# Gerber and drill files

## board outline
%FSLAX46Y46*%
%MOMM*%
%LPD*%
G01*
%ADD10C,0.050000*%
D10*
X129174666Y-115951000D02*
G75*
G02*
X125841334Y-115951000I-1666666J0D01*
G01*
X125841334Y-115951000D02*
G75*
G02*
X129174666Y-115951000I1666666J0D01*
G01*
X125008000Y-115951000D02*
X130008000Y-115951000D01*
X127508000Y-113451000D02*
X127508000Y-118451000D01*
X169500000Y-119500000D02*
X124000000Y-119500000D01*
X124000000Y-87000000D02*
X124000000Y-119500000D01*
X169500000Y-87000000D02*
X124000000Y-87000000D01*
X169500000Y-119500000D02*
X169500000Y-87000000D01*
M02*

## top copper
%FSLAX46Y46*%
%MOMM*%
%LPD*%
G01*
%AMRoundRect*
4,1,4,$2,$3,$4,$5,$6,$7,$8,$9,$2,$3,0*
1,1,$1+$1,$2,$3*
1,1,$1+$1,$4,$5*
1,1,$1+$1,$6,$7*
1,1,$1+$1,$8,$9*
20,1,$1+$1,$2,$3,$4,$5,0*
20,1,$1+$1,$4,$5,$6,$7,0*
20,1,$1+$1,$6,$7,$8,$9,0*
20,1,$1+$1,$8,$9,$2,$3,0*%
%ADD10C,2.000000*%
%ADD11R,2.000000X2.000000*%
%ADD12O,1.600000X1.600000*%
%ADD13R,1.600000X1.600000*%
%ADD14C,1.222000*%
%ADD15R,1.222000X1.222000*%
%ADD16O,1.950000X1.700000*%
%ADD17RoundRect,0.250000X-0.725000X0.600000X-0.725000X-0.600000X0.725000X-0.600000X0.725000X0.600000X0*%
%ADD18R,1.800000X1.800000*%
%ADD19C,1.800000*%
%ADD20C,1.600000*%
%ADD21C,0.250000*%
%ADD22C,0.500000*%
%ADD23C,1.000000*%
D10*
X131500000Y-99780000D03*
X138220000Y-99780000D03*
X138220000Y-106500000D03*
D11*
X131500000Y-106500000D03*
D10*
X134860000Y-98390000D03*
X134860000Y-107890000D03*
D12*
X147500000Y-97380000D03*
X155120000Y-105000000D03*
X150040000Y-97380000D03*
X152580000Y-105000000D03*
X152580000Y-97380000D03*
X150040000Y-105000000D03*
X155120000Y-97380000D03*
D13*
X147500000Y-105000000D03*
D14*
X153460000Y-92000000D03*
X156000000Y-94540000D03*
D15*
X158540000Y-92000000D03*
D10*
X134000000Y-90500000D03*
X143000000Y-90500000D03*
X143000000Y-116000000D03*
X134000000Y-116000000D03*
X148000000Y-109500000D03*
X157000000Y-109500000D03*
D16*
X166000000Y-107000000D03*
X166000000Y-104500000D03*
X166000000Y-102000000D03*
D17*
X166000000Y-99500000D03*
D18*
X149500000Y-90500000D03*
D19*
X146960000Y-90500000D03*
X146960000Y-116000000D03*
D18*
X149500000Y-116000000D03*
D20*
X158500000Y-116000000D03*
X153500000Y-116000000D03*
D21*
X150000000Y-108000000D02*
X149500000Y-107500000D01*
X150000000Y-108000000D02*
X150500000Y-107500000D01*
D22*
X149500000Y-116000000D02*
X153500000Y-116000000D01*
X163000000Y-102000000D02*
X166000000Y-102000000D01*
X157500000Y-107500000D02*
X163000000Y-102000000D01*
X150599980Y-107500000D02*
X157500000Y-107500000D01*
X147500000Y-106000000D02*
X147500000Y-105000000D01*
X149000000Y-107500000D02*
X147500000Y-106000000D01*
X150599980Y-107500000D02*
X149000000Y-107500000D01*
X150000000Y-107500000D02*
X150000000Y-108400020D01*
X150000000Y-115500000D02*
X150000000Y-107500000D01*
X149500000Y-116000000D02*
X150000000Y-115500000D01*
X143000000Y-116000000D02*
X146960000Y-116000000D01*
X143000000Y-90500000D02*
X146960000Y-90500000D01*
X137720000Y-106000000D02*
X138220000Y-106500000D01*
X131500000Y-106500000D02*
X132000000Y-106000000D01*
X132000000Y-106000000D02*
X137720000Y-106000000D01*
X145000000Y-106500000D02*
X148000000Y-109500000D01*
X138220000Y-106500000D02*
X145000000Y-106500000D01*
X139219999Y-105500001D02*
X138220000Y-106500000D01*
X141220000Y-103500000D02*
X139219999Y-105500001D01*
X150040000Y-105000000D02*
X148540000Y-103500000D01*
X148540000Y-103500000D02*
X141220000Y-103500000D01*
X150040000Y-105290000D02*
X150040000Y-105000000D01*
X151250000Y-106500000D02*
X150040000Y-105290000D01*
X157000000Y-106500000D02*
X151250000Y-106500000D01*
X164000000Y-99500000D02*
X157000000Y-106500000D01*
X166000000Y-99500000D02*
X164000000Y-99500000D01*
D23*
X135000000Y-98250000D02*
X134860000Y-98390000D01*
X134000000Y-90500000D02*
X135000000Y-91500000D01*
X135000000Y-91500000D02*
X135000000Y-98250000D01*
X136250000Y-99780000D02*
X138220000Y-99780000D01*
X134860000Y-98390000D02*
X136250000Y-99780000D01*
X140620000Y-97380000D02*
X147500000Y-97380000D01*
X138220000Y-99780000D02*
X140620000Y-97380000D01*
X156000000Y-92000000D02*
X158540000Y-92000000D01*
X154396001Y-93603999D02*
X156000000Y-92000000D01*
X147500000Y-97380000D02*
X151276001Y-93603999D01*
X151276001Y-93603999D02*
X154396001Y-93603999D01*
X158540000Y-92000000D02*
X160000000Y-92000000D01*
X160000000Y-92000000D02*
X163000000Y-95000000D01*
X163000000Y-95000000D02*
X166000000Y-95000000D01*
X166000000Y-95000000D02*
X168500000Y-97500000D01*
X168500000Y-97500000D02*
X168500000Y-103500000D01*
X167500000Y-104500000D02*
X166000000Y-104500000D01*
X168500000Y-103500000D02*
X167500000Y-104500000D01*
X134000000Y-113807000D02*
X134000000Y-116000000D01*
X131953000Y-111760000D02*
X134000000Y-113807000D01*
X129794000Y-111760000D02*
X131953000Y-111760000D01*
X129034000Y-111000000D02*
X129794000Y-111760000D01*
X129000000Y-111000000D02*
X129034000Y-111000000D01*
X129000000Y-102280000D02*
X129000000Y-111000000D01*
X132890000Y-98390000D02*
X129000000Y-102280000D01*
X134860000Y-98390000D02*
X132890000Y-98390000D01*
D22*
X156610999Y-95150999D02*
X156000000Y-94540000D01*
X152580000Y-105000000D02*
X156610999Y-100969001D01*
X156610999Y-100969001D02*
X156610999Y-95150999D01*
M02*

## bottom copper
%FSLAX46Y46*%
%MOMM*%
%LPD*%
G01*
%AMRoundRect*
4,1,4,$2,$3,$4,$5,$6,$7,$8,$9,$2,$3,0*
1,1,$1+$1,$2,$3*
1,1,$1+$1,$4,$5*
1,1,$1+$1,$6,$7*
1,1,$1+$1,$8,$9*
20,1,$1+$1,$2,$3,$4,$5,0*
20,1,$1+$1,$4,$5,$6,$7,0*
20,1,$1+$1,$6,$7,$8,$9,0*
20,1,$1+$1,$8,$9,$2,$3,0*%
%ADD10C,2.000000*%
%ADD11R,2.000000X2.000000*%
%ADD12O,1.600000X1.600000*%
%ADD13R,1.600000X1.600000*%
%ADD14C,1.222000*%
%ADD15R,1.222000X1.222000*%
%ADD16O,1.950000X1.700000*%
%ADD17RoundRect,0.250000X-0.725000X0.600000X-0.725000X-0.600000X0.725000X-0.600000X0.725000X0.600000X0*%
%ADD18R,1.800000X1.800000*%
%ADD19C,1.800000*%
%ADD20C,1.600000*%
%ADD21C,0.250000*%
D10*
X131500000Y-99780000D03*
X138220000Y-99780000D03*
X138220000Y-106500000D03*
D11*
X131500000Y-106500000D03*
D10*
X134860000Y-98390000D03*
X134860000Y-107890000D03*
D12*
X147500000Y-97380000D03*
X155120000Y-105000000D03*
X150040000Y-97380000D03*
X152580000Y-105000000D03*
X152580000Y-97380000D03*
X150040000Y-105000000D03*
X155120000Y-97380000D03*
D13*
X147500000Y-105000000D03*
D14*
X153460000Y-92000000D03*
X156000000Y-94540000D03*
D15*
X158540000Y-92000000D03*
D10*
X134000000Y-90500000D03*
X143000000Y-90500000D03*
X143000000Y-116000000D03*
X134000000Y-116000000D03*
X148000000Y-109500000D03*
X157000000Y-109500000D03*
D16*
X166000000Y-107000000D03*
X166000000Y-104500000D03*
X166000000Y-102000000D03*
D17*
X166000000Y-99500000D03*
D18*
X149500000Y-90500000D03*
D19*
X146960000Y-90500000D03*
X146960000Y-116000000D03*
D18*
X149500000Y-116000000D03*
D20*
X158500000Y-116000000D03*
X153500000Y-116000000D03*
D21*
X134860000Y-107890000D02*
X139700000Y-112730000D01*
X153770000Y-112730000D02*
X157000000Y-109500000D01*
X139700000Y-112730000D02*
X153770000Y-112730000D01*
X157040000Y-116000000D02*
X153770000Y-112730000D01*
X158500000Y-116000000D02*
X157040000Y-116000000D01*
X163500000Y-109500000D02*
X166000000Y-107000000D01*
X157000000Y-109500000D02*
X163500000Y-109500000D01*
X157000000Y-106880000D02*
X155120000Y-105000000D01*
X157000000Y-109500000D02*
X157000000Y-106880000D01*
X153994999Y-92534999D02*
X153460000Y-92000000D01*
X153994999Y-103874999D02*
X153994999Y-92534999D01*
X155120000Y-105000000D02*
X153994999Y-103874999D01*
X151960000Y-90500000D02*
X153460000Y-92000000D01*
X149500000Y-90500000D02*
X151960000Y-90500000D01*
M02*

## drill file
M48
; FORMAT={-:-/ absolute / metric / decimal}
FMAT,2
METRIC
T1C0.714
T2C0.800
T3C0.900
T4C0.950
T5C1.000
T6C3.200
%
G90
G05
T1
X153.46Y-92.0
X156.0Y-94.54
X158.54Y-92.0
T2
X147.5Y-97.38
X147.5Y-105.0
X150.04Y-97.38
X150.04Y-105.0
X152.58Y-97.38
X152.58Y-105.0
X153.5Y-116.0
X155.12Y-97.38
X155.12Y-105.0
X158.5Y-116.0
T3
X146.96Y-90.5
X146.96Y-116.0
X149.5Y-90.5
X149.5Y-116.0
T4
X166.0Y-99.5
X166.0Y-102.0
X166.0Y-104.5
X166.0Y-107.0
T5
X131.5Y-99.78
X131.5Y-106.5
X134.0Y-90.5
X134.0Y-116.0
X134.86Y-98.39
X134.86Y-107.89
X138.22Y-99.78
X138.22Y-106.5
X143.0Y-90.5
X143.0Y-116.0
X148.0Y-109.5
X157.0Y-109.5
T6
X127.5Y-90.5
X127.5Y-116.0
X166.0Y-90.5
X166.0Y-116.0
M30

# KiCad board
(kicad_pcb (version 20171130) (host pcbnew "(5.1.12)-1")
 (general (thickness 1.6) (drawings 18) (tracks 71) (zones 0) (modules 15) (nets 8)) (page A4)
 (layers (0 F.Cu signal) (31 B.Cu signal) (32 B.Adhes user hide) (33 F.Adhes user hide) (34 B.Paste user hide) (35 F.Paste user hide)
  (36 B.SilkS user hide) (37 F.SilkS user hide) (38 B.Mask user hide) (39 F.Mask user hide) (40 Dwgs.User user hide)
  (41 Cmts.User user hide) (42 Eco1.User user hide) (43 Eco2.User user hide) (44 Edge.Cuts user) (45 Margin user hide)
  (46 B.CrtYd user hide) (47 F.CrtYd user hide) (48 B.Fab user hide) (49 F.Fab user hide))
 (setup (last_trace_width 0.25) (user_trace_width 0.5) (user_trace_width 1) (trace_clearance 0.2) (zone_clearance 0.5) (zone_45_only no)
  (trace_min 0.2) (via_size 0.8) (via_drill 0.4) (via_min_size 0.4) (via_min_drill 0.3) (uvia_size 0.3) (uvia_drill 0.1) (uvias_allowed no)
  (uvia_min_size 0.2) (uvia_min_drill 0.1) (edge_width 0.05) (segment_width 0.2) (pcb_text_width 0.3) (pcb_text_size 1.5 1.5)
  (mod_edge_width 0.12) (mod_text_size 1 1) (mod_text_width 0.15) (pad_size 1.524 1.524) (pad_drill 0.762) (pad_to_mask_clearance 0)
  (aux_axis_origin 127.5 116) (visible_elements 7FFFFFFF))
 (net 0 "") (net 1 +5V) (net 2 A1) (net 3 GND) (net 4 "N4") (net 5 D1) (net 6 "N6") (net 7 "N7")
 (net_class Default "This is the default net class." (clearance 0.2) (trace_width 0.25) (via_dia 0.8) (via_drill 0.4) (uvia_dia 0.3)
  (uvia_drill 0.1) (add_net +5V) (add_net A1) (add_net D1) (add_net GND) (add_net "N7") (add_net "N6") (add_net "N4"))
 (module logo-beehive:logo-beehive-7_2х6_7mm (layer F.Cu) (at 161 113.5 90)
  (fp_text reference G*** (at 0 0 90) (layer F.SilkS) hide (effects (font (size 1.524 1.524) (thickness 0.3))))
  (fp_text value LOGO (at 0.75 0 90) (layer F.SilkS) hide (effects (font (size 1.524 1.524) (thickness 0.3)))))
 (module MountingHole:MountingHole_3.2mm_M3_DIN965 (layer F.Cu) (at 166 90.5)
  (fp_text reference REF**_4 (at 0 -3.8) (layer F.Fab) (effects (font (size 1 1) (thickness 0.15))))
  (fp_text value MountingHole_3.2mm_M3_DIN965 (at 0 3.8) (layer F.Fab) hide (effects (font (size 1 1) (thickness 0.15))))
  (pad 1 np_thru_hole circle (at 0 0) (size 3.2 3.2) (drill 3.2) (layers *.Cu *.Mask)))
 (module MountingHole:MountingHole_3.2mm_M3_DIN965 (layer F.Cu) (at 166 116)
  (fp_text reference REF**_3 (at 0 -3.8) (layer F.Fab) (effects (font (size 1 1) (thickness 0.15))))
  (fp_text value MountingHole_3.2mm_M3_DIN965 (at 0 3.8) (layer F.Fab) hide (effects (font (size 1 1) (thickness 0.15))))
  (pad 1 np_thru_hole circle (at 0 0) (size 3.2 3.2) (drill 3.2) (layers *.Cu *.Mask)))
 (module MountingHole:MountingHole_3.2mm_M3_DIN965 (layer F.Cu) (at 127.5 90.5)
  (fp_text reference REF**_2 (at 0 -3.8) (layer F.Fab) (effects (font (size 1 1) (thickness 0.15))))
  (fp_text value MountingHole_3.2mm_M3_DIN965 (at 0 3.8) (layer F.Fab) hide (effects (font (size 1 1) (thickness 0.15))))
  (pad 1 np_thru_hole circle (at 0 0) (size 3.2 3.2) (drill 3.2) (layers *.Cu *.Mask)))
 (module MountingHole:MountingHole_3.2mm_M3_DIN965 (layer F.Cu) (at 127.5 116)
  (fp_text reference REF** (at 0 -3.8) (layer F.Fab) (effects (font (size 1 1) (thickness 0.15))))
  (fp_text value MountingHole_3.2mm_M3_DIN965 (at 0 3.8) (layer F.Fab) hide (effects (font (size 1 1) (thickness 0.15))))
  (pad 1 np_thru_hole circle (at 0 0) (size 3.2 3.2) (drill 3.2) (layers *.Cu *.Mask)))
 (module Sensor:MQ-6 (layer F.Cu) (at 131.5 106.5 90)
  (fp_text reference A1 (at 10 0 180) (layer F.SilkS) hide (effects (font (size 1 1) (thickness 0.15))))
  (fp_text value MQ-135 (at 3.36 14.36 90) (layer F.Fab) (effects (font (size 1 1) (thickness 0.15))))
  (pad 6 thru_hole circle (at 6.72 0) (size 2 2) (drill 1) (layers *.Cu *.Mask) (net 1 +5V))
  (pad 4 thru_hole circle (at 6.72 6.72 270) (size 2 2) (drill 1) (layers *.Cu *.Mask) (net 1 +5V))
  (pad 3 thru_hole circle (at 0 6.72 180) (size 2 2) (drill 1) (layers *.Cu *.Mask) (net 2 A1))
  (pad 1 thru_hole rect (at 0 0 90) (size 2 2) (drill 1) (layers *.Cu *.Mask) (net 2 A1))
  (pad 5 thru_hole circle (at 8.11 3.36 90) (size 2 2) (drill 1) (layers *.Cu *.Mask) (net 1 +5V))
  (pad 2 thru_hole circle (at -1.39 3.36 90) (size 2 2) (drill 1) (layers *.Cu *.Mask) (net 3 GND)))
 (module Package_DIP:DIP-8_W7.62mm (layer F.Cu) (at 147.5 105 90)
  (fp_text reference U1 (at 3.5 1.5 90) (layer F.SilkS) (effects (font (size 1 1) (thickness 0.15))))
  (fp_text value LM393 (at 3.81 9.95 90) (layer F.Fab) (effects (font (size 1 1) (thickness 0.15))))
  (pad 8 thru_hole oval (at 7.62 0 90) (size 1.6 1.6) (drill 0.8) (layers *.Cu *.Mask) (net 1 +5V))
  (pad 4 thru_hole oval (at 0 7.62 90) (size 1.6 1.6) (drill 0.8) (layers *.Cu *.Mask) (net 3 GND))
  (pad 7 thru_hole oval (at 7.62 2.54 90) (size 1.6 1.6) (drill 0.8) (layers *.Cu *.Mask))
  (pad 3 thru_hole oval (at 0 5.08 90) (size 1.6 1.6) (drill 0.8) (layers *.Cu *.Mask) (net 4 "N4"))
  (pad 6 thru_hole oval (at 7.62 5.08 90) (size 1.6 1.6) (drill 0.8) (layers *.Cu *.Mask))
  (pad 2 thru_hole oval (at 0 2.54 90) (size 1.6 1.6) (drill 0.8) (layers *.Cu *.Mask) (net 2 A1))
  (pad 5 thru_hole oval (at 7.62 7.62 90) (size 1.6 1.6) (drill 0.8) (layers *.Cu *.Mask))
  (pad 1 thru_hole rect (at 0 0 90) (size 1.6 1.6) (drill 0.8) (layers *.Cu *.Mask) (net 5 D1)))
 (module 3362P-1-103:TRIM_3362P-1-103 (layer F.Cu) (at 156 92 180)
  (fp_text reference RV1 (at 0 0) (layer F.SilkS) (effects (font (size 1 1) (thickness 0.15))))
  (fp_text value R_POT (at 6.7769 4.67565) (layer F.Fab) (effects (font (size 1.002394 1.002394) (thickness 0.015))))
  (pad 3 thru_hole circle (at 2.54 0 180) (size 1.222 1.222) (drill 0.714) (layers *.Cu *.Mask) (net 3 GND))
  (pad 2 thru_hole circle (at 0 -2.54 180) (size 1.222 1.222) (drill 0.714) (layers *.Cu *.Mask) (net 4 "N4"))
  (pad 1 thru_hole rect (at -2.54 0 180) (size 1.222 1.222) (drill 0.714) (layers *.Cu *.Mask) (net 1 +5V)))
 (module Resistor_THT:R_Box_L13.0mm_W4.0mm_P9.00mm (layer F.Cu) (at 134 90.5)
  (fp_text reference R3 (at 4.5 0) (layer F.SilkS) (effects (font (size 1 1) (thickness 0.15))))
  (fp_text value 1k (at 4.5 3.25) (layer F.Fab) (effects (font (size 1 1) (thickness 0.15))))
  (pad 1 thru_hole circle (at 0 0) (size 2 2) (drill 1) (layers *.Cu *.Mask) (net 1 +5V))
  (pad 2 thru_hole circle (at 9 0) (size 2 2) (drill 1) (layers *.Cu *.Mask) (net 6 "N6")))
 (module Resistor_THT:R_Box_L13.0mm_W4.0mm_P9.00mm (layer F.Cu) (at 134 116)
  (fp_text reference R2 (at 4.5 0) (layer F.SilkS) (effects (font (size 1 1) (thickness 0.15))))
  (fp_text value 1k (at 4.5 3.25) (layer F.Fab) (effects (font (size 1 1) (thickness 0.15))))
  (pad 2 thru_hole circle (at 9 0) (size 2 2) (drill 1) (layers *.Cu *.Mask) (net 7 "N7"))
  (pad 1 thru_hole circle (at 0 0) (size 2 2) (drill 1) (layers *.Cu *.Mask) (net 1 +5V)))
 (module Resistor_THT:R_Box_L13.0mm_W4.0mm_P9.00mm (layer F.Cu) (at 148 109.5)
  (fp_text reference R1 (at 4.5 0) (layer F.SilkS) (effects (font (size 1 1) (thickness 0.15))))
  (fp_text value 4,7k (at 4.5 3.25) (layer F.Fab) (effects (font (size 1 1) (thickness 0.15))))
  (pad 1 thru_hole circle (at 0 0) (size 2 2) (drill 1) (layers *.Cu *.Mask) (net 2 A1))
  (pad 2 thru_hole circle (at 9 0) (size 2 2) (drill 1) (layers *.Cu *.Mask) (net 3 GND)))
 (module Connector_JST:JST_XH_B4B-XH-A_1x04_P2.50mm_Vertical (layer F.Cu) (at 166 99.5 270)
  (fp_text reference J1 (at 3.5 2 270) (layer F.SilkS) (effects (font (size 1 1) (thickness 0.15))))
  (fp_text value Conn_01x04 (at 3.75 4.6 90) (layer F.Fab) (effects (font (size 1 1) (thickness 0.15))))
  (pad 4 thru_hole oval (at 7.5 0 270) (size 1.7 1.95) (drill 0.95) (layers *.Cu *.Mask) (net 3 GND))
  (pad 3 thru_hole oval (at 5 0 270) (size 1.7 1.95) (drill 0.95) (layers *.Cu *.Mask) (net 1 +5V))
  (pad 2 thru_hole oval (at 2.5 0 270) (size 1.7 1.95) (drill 0.95) (layers *.Cu *.Mask) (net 5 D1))
  (pad 1 thru_hole roundrect (at 0 0 270) (size 1.7 1.95) (drill 0.95) (layers *.Cu *.Mask) (roundrect_rratio 0.1470588235294118) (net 2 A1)))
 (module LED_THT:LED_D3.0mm (layer F.Cu) (at 149.5 90.5 180)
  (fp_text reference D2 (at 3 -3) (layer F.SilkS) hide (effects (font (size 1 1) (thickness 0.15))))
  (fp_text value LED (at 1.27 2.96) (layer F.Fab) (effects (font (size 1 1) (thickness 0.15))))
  (pad 1 thru_hole rect (at 0 0 180) (size 1.8 1.8) (drill 0.9) (layers *.Cu *.Mask) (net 3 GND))
  (pad 2 thru_hole circle (at 2.54 0 180) (size 1.8 1.8) (drill 0.9) (layers *.Cu *.Mask) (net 6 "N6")))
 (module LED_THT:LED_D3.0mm (layer F.Cu) (at 149.5 116 180)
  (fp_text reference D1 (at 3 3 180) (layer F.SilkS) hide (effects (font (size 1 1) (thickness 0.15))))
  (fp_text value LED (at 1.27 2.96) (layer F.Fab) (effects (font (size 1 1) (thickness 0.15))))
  (pad 2 thru_hole circle (at 2.54 0 180) (size 1.8 1.8) (drill 0.9) (layers *.Cu *.Mask) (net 7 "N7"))
  (pad 1 thru_hole rect (at 0 0 180) (size 1.8 1.8) (drill 0.9) (layers *.Cu *.Mask) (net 5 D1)))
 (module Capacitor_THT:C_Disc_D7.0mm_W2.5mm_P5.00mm (layer F.Cu) (at 153.5 116)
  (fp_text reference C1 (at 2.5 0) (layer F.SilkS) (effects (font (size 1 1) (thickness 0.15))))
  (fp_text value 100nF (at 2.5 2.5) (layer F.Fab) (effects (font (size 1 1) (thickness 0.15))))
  (pad 2 thru_hole circle (at 5 0) (size 1.6 1.6) (drill 0.8) (layers *.Cu *.Mask) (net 3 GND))
  (pad 1 thru_hole circle (at 0 0) (size 1.6 1.6) (drill 0.8) (layers *.Cu *.Mask) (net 5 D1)))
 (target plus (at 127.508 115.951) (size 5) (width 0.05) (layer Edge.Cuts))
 (gr_line (start 169.5 119.5) (end 124 119.5) (layer Edge.Cuts) (width 0.05))
 (gr_line (start 124 87) (end 124 119.5) (layer Edge.Cuts) (width 0.05))
 (gr_line (start 169.5 87) (end 124 87) (layer Edge.Cuts) (width 0.05))
 (gr_line (start 169.5 119.5) (end 169.5 87) (layer Edge.Cuts) (width 0.05))
 (segment (start 134.86 107.89) (end 139.7 112.73) (width 0.25) (layer B.Cu) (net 3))
 (segment (start 153.77 112.73) (end 157 109.5) (width 0.25) (layer B.Cu) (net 3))
 (segment (start 139.7 112.73) (end 153.77 112.73) (width 0.25) (layer B.Cu) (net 3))
 (segment (start 157.04 116) (end 153.77 112.73) (width 0.25) (layer B.Cu) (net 3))
 (segment (start 158.5 116) (end 157.04 116) (width 0.25) (layer B.Cu) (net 3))
 (segment (start 163.5 109.5) (end 166 107) (width 0.25) (layer B.Cu) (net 3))
 (segment (start 157 109.5) (end 163.5 109.5) (width 0.25) (layer B.Cu) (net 3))
 (segment (start 157 106.88) (end 155.12 105) (width 0.25) (layer B.Cu) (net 3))
 (segment (start 157 109.5) (end 157 106.88) (width 0.25) (layer B.Cu) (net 3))
 (segment (start 153.994999 92.534999) (end 153.46 92) (width 0.25) (layer B.Cu) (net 3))
 (segment (start 153.994999 103.874999) (end 153.994999 92.534999) (width 0.25) (layer B.Cu) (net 3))
 (segment (start 155.12 105) (end 153.994999 103.874999) (width 0.25) (layer B.Cu) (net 3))
 (segment (start 151.96 90.5) (end 153.46 92) (width 0.25) (layer B.Cu) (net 3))
 (segment (start 149.5 90.5) (end 151.96 90.5) (width 0.25) (layer B.Cu) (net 3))
 (segment (start 150 108) (end 149.5 107.5) (width 0.25) (layer F.Cu) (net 5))
 (segment (start 150 108) (end 150.5 107.5) (width 0.25) (layer F.Cu) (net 5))
 (segment (start 149.5 116) (end 153.5 116) (width 0.5) (layer F.Cu) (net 5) (status 30))
 (segment (start 163 102) (end 166 102) (width 0.5) (layer F.Cu) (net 5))
 (segment (start 157.5 107.5) (end 163 102) (width 0.5) (layer F.Cu) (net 5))
 (segment (start 150.59998 107.5) (end 157.5 107.5) (width 0.5) (layer F.Cu) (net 5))
 (segment (start 147.5 106) (end 147.5 105) (width 0.5) (layer F.Cu) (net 5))
 (segment (start 149 107.5) (end 147.5 106) (width 0.5) (layer F.Cu) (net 5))
 (segment (start 150.59998 107.5) (end 149 107.5) (width 0.5) (layer F.Cu) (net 5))
 (segment (start 150 107.5) (end 150 108.40002) (width 0.5) (layer F.Cu) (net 5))
 (segment (start 150 115.5) (end 150 107.5) (width 0.5) (layer F.Cu) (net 5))
 (segment (start 149.5 116) (end 150 115.5) (width 0.5) (layer F.Cu) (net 5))
 (segment (start 143 116) (end 146.96 116) (width 0.5) (layer F.Cu) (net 7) (status 30))
 (segment (start 143 90.5) (end 146.96 90.5) (width 0.5) (layer F.Cu) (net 6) (status 30))
 (segment (start 137.72 106) (end 138.22 106.5) (width 0.5) (layer F.Cu) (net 2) (status 30))
 (segment (start 131.5 106.5) (end 132 106) (width 0.5) (layer F.Cu) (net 2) (status 30))
 (segment (start 132 106) (end 137.72 106) (width 0.5) (layer F.Cu) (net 2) (status 30))
 (segment (start 145 106.5) (end 148 109.5) (width 0.5) (layer F.Cu) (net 2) (status 20))
 (segment (start 138.22 106.5) (end 145 106.5) (width 0.5) (layer F.Cu) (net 2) (status 10))
 (segment (start 139.219999 105.500001) (end 138.22 106.5) (width 0.5) (layer F.Cu) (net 2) (status 20))
 (segment (start 141.22 103.5) (end 139.219999 105.500001) (width 0.5) (layer F.Cu) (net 2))
 (segment (start 150.04 105) (end 148.54 103.5) (width 0.5) (layer F.Cu) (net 2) (status 10))
 (segment (start 148.54 103.5) (end 141.22 103.5) (width 0.5) (layer F.Cu) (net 2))
 (segment (start 150.04 105.29) (end 150.04 105) (width 0.5) (layer F.Cu) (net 2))
 (segment (start 151.25 106.5) (end 150.04 105.29) (width 0.5) (layer F.Cu) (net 2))
 (segment (start 157 106.5) (end 151.25 106.5) (width 0.5) (layer F.Cu) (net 2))
 (segment (start 164 99.5) (end 157 106.5) (width 0.5) (layer F.Cu) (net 2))
 (segment (start 166 99.5) (end 164 99.5) (width 0.5) (layer F.Cu) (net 2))
 (segment (start 135 98.25) (end 134.86 98.39) (width 1) (layer F.Cu) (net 1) (status 30))
 (segment (start 134 90.5) (end 135 91.5) (width 1) (layer F.Cu) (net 1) (status 10))
 (segment (start 135 91.5) (end 135 98.25) (width 1) (layer F.Cu) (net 1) (status 20))
 (segment (start 136.25 99.78) (end 138.22 99.78) (width 1) (layer F.Cu) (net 1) (status 20))
 (segment (start 134.86 98.39) (end 136.25 99.78) (width 1) (layer F.Cu) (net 1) (status 10))
 (segment (start 140.62 97.38) (end 147.5 97.38) (width 1) (layer F.Cu) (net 1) (status 20))
 (segment (start 138.22 99.78) (end 140.62 97.38) (width 1) (layer F.Cu) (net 1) (status 10))
 (segment (start 156 92) (end 158.54 92) (width 1) (layer F.Cu) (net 1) (status 20))
 (segment (start 154.396001 93.603999) (end 156 92) (width 1) (layer F.Cu) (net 1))
 (segment (start 147.5 97.38) (end 151.276001 93.603999) (width 1) (layer F.Cu) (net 1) (status 10))
 (segment (start 151.276001 93.603999) (end 154.396001 93.603999) (width 1) (layer F.Cu) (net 1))
 (segment (start 158.54 92) (end 160 92) (width 1) (layer F.Cu) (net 1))
 (segment (start 160 92) (end 163 95) (width 1) (layer F.Cu) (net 1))
 (segment (start 163 95) (end 166 95) (width 1) (layer F.Cu) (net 1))
 (segment (start 166 95) (end 168.5 97.5) (width 1) (layer F.Cu) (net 1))
 (segment (start 168.5 97.5) (end 168.5 103.5) (width 1) (layer F.Cu) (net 1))
 (segment (start 167.5 104.5) (end 166 104.5) (width 1) (layer F.Cu) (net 1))
 (segment (start 168.5 103.5) (end 167.5 104.5) (width 1) (layer F.Cu) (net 1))
 (segment (start 134 113.807) (end 134 116) (width 1) (layer F.Cu) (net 1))
 (segment (start 131.953 111.76) (end 134 113.807) (width 1) (layer F.Cu) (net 1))
 (segment (start 129.794 111.76) (end 131.953 111.76) (width 1) (layer F.Cu) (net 1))
 (segment (start 129.034 111) (end 129.794 111.76) (width 1) (layer F.Cu) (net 1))
 (segment (start 129 111) (end 129.034 111) (width 1) (layer F.Cu) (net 1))
 (segment (start 129 102.28) (end 129 111) (width 1) (layer F.Cu) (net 1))
 (segment (start 132.89 98.39) (end 129 102.28) (width 1) (layer F.Cu) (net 1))
 (segment (start 134.86 98.39) (end 132.89 98.39) (width 1) (layer F.Cu) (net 1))
 (segment (start 156.610999 95.150999) (end 156 94.54) (width 0.5) (layer F.Cu) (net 4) (status 20))
 (segment (start 152.58 105) (end 156.610999 100.969001) (width 0.5) (layer F.Cu) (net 4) (status 10))
 (segment (start 156.610999 100.969001) (end 156.610999 95.150999) (width 0.5) (layer F.Cu) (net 4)))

